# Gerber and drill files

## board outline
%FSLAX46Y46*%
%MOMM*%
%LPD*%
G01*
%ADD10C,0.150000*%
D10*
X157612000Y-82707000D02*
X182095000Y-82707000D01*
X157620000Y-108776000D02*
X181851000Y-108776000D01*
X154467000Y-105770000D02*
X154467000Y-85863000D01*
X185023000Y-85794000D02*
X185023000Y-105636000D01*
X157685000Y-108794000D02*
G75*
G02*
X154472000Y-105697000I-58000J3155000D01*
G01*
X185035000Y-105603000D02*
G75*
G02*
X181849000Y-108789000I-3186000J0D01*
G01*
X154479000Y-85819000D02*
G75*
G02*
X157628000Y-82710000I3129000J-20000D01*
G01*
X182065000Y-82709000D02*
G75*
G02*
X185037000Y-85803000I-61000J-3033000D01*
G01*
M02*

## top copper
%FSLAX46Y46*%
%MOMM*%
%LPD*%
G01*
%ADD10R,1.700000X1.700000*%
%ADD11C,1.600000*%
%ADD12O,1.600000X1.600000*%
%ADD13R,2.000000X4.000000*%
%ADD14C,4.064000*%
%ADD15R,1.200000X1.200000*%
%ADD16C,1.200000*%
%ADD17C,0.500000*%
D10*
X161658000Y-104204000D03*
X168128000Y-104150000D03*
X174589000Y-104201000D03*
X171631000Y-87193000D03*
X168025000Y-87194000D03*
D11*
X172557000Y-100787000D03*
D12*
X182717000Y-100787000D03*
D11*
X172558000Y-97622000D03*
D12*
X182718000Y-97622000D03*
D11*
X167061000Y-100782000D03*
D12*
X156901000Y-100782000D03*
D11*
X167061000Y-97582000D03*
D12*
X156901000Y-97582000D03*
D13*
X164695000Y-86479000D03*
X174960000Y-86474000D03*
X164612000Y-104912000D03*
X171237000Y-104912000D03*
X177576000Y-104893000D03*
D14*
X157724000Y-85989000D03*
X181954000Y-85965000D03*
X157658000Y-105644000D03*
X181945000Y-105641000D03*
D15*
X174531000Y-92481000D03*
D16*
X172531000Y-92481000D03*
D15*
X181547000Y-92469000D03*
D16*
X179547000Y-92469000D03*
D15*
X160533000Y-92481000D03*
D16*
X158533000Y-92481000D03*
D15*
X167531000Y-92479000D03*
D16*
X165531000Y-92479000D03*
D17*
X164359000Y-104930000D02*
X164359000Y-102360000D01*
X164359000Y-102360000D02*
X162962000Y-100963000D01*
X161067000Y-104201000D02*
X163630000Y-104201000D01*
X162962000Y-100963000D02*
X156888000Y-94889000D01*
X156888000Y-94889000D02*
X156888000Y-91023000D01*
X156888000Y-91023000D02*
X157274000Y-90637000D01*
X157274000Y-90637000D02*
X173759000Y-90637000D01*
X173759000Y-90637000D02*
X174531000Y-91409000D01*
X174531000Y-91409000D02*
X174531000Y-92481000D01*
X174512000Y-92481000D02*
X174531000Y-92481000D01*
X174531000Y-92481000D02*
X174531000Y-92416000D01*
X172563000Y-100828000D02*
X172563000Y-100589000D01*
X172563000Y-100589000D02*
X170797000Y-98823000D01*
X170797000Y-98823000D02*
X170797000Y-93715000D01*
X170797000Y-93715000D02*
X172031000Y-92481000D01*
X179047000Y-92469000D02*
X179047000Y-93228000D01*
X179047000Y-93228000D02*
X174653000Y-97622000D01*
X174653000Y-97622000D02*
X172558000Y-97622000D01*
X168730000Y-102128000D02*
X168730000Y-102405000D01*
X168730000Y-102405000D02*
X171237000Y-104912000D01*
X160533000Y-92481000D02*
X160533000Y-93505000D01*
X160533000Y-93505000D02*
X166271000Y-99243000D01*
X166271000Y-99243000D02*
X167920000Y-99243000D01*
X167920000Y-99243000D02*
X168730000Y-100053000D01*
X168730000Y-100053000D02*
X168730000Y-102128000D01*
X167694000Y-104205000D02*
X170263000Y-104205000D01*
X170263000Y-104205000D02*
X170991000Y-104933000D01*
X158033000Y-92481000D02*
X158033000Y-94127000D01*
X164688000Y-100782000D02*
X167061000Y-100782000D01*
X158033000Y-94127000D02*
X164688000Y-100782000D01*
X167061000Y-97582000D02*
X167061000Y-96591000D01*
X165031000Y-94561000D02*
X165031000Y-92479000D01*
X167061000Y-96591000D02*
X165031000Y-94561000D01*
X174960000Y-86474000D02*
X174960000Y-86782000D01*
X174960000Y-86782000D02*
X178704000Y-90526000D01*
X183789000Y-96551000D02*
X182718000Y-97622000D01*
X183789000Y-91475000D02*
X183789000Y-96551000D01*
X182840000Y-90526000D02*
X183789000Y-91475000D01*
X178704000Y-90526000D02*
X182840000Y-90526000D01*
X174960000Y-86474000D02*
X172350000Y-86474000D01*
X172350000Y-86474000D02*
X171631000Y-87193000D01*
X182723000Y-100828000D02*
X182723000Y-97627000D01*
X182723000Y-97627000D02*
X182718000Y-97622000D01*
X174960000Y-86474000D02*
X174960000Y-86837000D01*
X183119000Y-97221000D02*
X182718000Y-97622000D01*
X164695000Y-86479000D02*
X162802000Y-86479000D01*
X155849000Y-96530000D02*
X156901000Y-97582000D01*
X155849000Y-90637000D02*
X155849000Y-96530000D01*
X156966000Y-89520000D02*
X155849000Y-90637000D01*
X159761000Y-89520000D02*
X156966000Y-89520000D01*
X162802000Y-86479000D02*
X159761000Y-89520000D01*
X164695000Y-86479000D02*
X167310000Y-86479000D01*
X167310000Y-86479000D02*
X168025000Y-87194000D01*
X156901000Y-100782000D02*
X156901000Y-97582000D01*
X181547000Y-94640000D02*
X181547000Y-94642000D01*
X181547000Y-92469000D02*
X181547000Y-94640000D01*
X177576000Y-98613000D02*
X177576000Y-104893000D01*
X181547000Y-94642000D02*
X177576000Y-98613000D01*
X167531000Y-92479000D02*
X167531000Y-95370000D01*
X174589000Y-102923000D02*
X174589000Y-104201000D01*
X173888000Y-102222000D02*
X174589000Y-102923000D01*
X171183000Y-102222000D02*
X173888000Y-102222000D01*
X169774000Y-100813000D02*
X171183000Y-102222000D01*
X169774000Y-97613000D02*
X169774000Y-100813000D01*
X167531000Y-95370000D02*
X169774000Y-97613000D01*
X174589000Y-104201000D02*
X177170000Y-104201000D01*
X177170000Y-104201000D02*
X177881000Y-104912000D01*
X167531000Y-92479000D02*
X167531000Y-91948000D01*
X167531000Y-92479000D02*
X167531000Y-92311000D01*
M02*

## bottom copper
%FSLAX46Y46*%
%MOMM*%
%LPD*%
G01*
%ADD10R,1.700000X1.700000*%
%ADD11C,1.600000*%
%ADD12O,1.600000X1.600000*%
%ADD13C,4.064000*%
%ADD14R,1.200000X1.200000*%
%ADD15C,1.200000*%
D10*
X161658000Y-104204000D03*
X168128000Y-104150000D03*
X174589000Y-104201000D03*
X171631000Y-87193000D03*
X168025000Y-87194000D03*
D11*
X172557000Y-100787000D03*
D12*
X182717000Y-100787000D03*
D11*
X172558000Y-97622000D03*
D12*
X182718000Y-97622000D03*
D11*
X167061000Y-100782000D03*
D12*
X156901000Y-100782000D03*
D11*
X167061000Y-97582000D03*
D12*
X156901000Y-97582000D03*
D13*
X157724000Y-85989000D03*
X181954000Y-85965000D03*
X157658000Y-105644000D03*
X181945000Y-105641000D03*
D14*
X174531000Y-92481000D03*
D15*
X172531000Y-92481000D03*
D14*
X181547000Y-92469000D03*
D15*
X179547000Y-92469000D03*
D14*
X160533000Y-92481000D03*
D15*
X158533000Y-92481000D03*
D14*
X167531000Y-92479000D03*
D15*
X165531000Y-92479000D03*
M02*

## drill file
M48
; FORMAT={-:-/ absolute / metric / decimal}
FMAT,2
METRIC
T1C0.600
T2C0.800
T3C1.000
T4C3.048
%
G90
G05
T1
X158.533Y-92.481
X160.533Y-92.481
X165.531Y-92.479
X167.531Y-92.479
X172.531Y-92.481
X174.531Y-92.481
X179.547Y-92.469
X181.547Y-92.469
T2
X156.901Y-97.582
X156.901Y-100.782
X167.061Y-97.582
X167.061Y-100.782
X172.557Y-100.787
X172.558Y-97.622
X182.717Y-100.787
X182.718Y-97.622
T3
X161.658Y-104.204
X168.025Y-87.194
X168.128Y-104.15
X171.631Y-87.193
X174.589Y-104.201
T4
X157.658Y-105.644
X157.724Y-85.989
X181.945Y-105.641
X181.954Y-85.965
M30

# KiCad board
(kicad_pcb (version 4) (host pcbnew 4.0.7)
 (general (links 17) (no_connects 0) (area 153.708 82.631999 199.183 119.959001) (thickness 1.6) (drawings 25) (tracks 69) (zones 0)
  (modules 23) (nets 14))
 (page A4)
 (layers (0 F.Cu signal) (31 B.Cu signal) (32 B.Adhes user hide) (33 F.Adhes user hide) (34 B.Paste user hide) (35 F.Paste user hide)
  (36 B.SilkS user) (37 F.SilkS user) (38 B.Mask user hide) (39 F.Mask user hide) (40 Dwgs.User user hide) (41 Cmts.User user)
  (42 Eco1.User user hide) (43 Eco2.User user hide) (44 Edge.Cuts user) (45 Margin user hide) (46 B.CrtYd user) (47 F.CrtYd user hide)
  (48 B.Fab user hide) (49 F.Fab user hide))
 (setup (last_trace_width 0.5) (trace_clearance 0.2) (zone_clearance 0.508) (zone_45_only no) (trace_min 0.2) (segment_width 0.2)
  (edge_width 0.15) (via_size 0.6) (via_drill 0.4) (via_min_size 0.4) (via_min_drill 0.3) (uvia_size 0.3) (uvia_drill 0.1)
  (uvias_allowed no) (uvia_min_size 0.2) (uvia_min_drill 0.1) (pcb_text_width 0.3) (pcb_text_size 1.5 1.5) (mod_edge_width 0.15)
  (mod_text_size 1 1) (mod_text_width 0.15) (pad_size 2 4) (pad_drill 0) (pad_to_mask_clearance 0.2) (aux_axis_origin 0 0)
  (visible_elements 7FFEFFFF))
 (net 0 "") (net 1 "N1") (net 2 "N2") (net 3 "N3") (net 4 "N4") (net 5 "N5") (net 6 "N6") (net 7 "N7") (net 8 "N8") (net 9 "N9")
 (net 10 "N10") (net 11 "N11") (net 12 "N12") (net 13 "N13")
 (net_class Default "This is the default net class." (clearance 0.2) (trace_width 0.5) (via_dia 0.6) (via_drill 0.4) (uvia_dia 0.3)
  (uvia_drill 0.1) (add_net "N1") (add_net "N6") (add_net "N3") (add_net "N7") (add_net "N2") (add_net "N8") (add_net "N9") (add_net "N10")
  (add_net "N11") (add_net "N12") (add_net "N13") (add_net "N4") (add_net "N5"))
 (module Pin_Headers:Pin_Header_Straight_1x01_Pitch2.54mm (layer F.Cu) (at 161.658 104.204)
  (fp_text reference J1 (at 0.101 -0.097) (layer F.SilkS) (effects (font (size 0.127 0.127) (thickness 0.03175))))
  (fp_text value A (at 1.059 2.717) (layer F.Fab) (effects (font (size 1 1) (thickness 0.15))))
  (pad 1 thru_hole rect (at 0 0) (size 1.7 1.7) (drill 1) (layers *.Cu *.Mask) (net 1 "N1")))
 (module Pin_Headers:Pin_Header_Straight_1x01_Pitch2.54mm (layer F.Cu) (at 168.128 104.15)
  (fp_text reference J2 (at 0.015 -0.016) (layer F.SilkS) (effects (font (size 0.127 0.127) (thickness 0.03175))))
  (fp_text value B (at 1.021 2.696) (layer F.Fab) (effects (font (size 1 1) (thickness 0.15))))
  (pad 1 thru_hole rect (at 0 0) (size 1.7 1.7) (drill 1) (layers *.Cu *.Mask) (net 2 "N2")))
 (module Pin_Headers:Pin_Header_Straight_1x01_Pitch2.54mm (layer F.Cu) (at 174.589 104.201)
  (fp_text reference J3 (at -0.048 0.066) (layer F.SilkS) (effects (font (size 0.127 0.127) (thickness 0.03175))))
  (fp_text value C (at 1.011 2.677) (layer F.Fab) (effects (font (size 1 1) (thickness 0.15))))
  (pad 1 thru_hole rect (at 0 0) (size 1.7 1.7) (drill 1) (layers *.Cu *.Mask) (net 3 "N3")))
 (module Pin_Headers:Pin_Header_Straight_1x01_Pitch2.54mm (layer F.Cu) (at 171.631 87.193)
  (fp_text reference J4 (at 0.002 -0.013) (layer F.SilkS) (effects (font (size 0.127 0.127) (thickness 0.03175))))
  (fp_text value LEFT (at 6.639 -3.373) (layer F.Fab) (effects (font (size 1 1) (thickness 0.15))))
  (pad 1 thru_hole rect (at 0 0) (size 1.7 1.7) (drill 1) (layers *.Cu *.Mask) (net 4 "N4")))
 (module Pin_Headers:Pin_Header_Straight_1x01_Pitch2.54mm (layer F.Cu) (at 168.025 87.194)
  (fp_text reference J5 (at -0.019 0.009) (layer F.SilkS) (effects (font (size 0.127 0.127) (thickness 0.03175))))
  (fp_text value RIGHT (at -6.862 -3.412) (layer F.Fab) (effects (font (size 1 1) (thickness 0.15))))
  (pad 1 thru_hole rect (at 0 0) (size 1.7 1.7) (drill 1) (layers *.Cu *.Mask) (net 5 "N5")))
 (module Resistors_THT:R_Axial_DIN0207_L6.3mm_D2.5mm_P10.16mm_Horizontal (layer F.Cu) (at 172.557 100.787)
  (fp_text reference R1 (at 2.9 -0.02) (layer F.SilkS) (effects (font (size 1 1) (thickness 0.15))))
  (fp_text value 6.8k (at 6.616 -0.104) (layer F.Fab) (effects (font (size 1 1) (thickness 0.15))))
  (pad 1 thru_hole circle (at 0 0) (size 1.6 1.6) (drill 0.8) (layers *.Cu *.Mask) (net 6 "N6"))
  (pad 2 thru_hole oval (at 10.16 0) (size 1.6 1.6) (drill 0.8) (layers *.Cu *.Mask) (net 4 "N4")))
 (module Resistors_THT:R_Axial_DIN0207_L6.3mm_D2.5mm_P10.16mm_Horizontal (layer F.Cu) (at 172.558 97.622)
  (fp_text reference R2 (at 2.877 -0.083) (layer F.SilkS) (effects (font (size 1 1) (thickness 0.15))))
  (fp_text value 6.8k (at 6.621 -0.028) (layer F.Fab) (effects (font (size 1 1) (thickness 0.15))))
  (pad 1 thru_hole circle (at 0 0) (size 1.6 1.6) (drill 0.8) (layers *.Cu *.Mask) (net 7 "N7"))
  (pad 2 thru_hole oval (at 10.16 0) (size 1.6 1.6) (drill 0.8) (layers *.Cu *.Mask) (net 4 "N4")))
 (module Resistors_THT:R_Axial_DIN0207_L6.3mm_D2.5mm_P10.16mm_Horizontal (layer F.Cu) (at 167.061 100.782 180)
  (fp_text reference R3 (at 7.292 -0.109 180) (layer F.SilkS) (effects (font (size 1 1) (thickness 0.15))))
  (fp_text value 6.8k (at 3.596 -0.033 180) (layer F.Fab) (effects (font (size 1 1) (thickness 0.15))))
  (pad 1 thru_hole circle (at 0 0 180) (size 1.6 1.6) (drill 0.8) (layers *.Cu *.Mask) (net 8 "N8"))
  (pad 2 thru_hole oval (at 10.16 0 180) (size 1.6 1.6) (drill 0.8) (layers *.Cu *.Mask) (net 5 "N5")))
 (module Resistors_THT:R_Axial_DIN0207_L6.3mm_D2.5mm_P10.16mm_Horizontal (layer F.Cu) (at 167.061 97.582 180)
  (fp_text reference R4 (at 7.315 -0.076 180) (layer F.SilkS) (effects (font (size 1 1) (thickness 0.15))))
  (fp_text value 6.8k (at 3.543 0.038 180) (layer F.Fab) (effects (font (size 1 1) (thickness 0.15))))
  (pad 1 thru_hole circle (at 0 0 180) (size 1.6 1.6) (drill 0.8) (layers *.Cu *.Mask) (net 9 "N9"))
  (pad 2 thru_hole oval (at 10.16 0 180) (size 1.6 1.6) (drill 0.8) (layers *.Cu *.Mask) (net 5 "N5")))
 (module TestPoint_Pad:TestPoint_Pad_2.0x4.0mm (layer F.Cu) (at 164.695 86.479)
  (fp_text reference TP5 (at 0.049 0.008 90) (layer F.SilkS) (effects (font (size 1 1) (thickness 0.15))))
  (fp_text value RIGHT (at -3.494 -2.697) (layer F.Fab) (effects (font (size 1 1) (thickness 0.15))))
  (pad 1 smd rect (at 0 0) (size 2 4) (layers F.Cu F.Mask) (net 5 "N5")))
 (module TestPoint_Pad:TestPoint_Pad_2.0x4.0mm (layer F.Cu) (at 174.96 86.474)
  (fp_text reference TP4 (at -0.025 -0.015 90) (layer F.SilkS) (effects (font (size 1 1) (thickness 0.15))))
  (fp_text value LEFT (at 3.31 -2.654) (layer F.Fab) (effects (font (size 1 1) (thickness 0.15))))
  (pad 1 smd rect (at 0 0) (size 2 4) (layers F.Cu F.Mask) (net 4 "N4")))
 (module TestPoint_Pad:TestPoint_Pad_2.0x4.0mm (layer F.Cu) (at 164.612 104.912)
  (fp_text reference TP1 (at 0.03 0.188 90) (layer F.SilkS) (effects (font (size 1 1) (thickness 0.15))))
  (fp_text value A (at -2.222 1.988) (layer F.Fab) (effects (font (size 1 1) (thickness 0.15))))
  (pad 1 smd rect (at 0 0) (size 2 4) (layers F.Cu F.Mask) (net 1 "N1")))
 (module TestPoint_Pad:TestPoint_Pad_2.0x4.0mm (layer F.Cu) (at 171.237 104.912)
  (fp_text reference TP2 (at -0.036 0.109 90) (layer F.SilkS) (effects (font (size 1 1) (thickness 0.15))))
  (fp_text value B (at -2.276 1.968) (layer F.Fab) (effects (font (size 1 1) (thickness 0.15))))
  (pad 1 smd rect (at 0 0) (size 2 4) (layers F.Cu F.Mask) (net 2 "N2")))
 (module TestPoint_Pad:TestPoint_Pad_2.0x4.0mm (layer F.Cu) (at 177.576 104.893)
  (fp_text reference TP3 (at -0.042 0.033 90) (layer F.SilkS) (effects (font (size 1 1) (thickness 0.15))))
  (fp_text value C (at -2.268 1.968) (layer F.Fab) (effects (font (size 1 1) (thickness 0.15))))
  (pad 1 smd rect (at 0 0) (size 2 4) (layers F.Cu F.Mask) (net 3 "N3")))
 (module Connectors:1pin (layer F.Cu) (at 157.724 85.989)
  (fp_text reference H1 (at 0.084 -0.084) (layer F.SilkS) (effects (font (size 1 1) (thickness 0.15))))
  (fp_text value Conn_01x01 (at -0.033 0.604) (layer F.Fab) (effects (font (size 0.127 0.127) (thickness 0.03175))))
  (pad 1 thru_hole circle (at 0 0) (size 4.064 4.064) (drill 3.048) (layers *.Cu *.Mask) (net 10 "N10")))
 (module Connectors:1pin (layer F.Cu) (at 181.954 85.965)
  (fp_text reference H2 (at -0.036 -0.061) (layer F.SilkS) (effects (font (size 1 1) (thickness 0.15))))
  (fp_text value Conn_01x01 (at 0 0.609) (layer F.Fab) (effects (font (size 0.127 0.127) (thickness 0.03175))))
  (pad 1 thru_hole circle (at 0 0) (size 4.064 4.064) (drill 3.048) (layers *.Cu *.Mask) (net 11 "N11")))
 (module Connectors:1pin (layer F.Cu) (at 157.658 105.644)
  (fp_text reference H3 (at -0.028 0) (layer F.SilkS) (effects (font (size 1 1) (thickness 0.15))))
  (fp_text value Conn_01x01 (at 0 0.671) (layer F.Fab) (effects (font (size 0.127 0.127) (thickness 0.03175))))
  (pad 1 thru_hole circle (at 0 0) (size 4.064 4.064) (drill 3.048) (layers *.Cu *.Mask) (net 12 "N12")))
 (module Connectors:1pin (layer F.Cu) (at 181.945 105.641)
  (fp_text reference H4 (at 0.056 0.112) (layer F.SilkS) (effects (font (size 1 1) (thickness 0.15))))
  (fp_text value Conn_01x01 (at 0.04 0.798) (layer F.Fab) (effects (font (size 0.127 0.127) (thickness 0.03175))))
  (pad 1 thru_hole circle (at 0 0) (size 4.064 4.064) (drill 3.048) (layers *.Cu *.Mask) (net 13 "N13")))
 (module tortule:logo (layer B.Cu) (at 172.273 95.722 180)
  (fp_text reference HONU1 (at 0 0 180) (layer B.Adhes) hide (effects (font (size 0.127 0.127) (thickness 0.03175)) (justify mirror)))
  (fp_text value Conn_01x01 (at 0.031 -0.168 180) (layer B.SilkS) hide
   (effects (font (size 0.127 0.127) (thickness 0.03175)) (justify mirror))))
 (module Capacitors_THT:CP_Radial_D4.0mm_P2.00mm (layer F.Cu) (at 174.531 92.481 180)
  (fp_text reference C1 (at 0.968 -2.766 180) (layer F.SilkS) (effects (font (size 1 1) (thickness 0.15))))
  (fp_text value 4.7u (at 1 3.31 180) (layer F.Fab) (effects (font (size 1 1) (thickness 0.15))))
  (pad 1 thru_hole rect (at 0 0 180) (size 1.2 1.2) (drill 0.6) (layers *.Cu *.Mask) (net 1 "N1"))
  (pad 2 thru_hole circle (at 2 0 180) (size 1.2 1.2) (drill 0.6) (layers *.Cu *.Mask) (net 6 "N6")))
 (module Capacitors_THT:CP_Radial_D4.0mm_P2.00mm (layer F.Cu) (at 181.547 92.469 180)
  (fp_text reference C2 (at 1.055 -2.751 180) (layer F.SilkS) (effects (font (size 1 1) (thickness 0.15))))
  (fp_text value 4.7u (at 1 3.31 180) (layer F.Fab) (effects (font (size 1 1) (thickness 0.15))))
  (pad 1 thru_hole rect (at 0 0 180) (size 1.2 1.2) (drill 0.6) (layers *.Cu *.Mask) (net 3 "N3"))
  (pad 2 thru_hole circle (at 2 0 180) (size 1.2 1.2) (drill 0.6) (layers *.Cu *.Mask) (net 7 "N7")))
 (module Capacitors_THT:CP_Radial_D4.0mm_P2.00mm (layer F.Cu) (at 160.533 92.481 180)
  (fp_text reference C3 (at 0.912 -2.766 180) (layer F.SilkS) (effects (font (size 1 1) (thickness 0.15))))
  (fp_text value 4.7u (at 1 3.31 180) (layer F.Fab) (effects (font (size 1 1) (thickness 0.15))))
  (pad 1 thru_hole rect (at 0 0 180) (size 1.2 1.2) (drill 0.6) (layers *.Cu *.Mask) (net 2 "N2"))
  (pad 2 thru_hole circle (at 2 0 180) (size 1.2 1.2) (drill 0.6) (layers *.Cu *.Mask) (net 8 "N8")))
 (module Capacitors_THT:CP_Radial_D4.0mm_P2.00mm (layer F.Cu) (at 167.531 92.479 180)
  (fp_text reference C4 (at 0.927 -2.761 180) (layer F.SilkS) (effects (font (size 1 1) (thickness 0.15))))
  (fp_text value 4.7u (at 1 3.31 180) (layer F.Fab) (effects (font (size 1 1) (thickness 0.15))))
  (pad 1 thru_hole rect (at 0 0 180) (size 1.2 1.2) (drill 0.6) (layers *.Cu *.Mask) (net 3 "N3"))
  (pad 2 thru_hole circle (at 2 0 180) (size 1.2 1.2) (drill 0.6) (layers *.Cu *.Mask) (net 9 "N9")))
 (gr_line (start 157.612 82.707) (end 182.095 82.707) (angle 90) (layer Edge.Cuts) (width 0.15))
 (gr_line (start 157.62 108.776) (end 181.851 108.776) (angle 90) (layer Edge.Cuts) (width 0.15))
 (gr_line (start 154.467 105.77) (end 154.467 85.863) (angle 90) (layer Edge.Cuts) (width 0.15))
 (gr_line (start 185.023 85.794) (end 185.023 105.636) (angle 90) (layer Edge.Cuts) (width 0.15))
 (gr_arc (start 157.627 105.639) (end 157.685 108.794) (angle 90) (layer Edge.Cuts) (width 0.15))
 (gr_arc (start 181.849 105.603) (end 185.035 105.603) (angle 90) (layer Edge.Cuts) (width 0.15))
 (gr_arc (start 157.608 85.839) (end 154.479 85.819) (angle 90) (layer Edge.Cuts) (width 0.15))
 (gr_arc (start 182.004 85.742) (end 182.065 82.709) (angle 90) (layer Edge.Cuts) (width 0.15))
 (segment (start 164.359 104.93) (end 164.359 102.36) (width 0.5) (layer F.Cu) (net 1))
 (segment (start 164.359 102.36) (end 162.962 100.963) (width 0.5) (layer F.Cu) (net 1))
 (segment (start 161.067 104.201) (end 163.63 104.201) (width 0.5) (layer F.Cu) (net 1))
 (segment (start 162.962 100.963) (end 156.888 94.889) (width 0.5) (layer F.Cu) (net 1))
 (segment (start 156.888 94.889) (end 156.888 91.023) (width 0.5) (layer F.Cu) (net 1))
 (segment (start 156.888 91.023) (end 157.274 90.637) (width 0.5) (layer F.Cu) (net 1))
 (segment (start 157.274 90.637) (end 173.759 90.637) (width 0.5) (layer F.Cu) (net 1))
 (segment (start 173.759 90.637) (end 174.531 91.409) (width 0.5) (layer F.Cu) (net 1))
 (segment (start 174.531 91.409) (end 174.531 92.481) (width 0.5) (layer F.Cu) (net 1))
 (segment (start 174.512 92.481) (end 174.531 92.481) (width 0.5) (layer F.Cu) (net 1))
 (segment (start 174.531 92.481) (end 174.531 92.416) (width 0.5) (layer F.Cu) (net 1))
 (segment (start 172.563 100.828) (end 172.563 100.589) (width 0.5) (layer F.Cu) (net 6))
 (segment (start 172.563 100.589) (end 170.797 98.823) (width 0.5) (layer F.Cu) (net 6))
 (segment (start 170.797 98.823) (end 170.797 93.715) (width 0.5) (layer F.Cu) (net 6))
 (segment (start 170.797 93.715) (end 172.031 92.481) (width 0.5) (layer F.Cu) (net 6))
 (segment (start 179.047 92.469) (end 179.047 93.228) (width 0.5) (layer F.Cu) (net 7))
 (segment (start 179.047 93.228) (end 174.653 97.622) (width 0.5) (layer F.Cu) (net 7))
 (segment (start 174.653 97.622) (end 172.558 97.622) (width 0.5) (layer F.Cu) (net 7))
 (segment (start 168.73 102.128) (end 168.73 102.405) (width 0.5) (layer F.Cu) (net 2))
 (segment (start 168.73 102.405) (end 171.237 104.912) (width 0.5) (layer F.Cu) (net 2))
 (segment (start 160.533 92.481) (end 160.533 93.505) (width 0.5) (layer F.Cu) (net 2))
 (segment (start 160.533 93.505) (end 166.271 99.243) (width 0.5) (layer F.Cu) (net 2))
 (segment (start 166.271 99.243) (end 167.92 99.243) (width 0.5) (layer F.Cu) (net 2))
 (segment (start 167.92 99.243) (end 168.73 100.053) (width 0.5) (layer F.Cu) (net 2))
 (segment (start 168.73 100.053) (end 168.73 102.128) (width 0.5) (layer F.Cu) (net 2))
 (segment (start 167.694 104.205) (end 170.263 104.205) (width 0.5) (layer F.Cu) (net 2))
 (segment (start 170.263 104.205) (end 170.991 104.933) (width 0.5) (layer F.Cu) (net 2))
 (segment (start 158.033 92.481) (end 158.033 94.127) (width 0.5) (layer F.Cu) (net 8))
 (segment (start 164.688 100.782) (end 167.061 100.782) (width 0.5) (layer F.Cu) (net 8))
 (segment (start 158.033 94.127) (end 164.688 100.782) (width 0.5) (layer F.Cu) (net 8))
 (segment (start 167.061 97.582) (end 167.061 96.591) (width 0.5) (layer F.Cu) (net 9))
 (segment (start 165.031 94.561) (end 165.031 92.479) (width 0.5) (layer F.Cu) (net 9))
 (segment (start 167.061 96.591) (end 165.031 94.561) (width 0.5) (layer F.Cu) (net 9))
 (segment (start 174.96 86.474) (end 174.96 86.782) (width 0.5) (layer F.Cu) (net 4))
 (segment (start 174.96 86.782) (end 178.704 90.526) (width 0.5) (layer F.Cu) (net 4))
 (segment (start 183.789 96.551) (end 182.718 97.622) (width 0.5) (layer F.Cu) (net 4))
 (segment (start 183.789 91.475) (end 183.789 96.551) (width 0.5) (layer F.Cu) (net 4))
 (segment (start 182.84 90.526) (end 183.789 91.475) (width 0.5) (layer F.Cu) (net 4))
 (segment (start 178.704 90.526) (end 182.84 90.526) (width 0.5) (layer F.Cu) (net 4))
 (segment (start 174.96 86.474) (end 172.35 86.474) (width 0.5) (layer F.Cu) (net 4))
 (segment (start 172.35 86.474) (end 171.631 87.193) (width 0.5) (layer F.Cu) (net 4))
 (segment (start 182.723 100.828) (end 182.723 97.627) (width 0.5) (layer F.Cu) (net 4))
 (segment (start 182.723 97.627) (end 182.718 97.622) (width 0.5) (layer F.Cu) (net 4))
 (segment (start 174.96 86.474) (end 174.96 86.837) (width 0.5) (layer F.Cu) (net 4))
 (segment (start 183.119 97.221) (end 182.718 97.622) (width 0.5) (layer F.Cu) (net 4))
 (segment (start 164.695 86.479) (end 162.802 86.479) (width 0.5) (layer F.Cu) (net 5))
 (segment (start 155.849 96.53) (end 156.901 97.582) (width 0.5) (layer F.Cu) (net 5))
 (segment (start 155.849 90.637) (end 155.849 96.53) (width 0.5) (layer F.Cu) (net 5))
 (segment (start 156.966 89.52) (end 155.849 90.637) (width 0.5) (layer F.Cu) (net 5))
 (segment (start 159.761 89.52) (end 156.966 89.52) (width 0.5) (layer F.Cu) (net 5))
 (segment (start 162.802 86.479) (end 159.761 89.52) (width 0.5) (layer F.Cu) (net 5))
 (segment (start 164.695 86.479) (end 167.31 86.479) (width 0.5) (layer F.Cu) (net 5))
 (segment (start 167.31 86.479) (end 168.025 87.194) (width 0.5) (layer F.Cu) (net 5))
 (segment (start 156.901 100.782) (end 156.901 97.582) (width 0.5) (layer F.Cu) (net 5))
 (segment (start 181.547 94.64) (end 181.547 94.642) (width 0.5) (layer F.Cu) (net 3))
 (segment (start 181.547 92.469) (end 181.547 94.64) (width 0.5) (layer F.Cu) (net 3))
 (segment (start 177.576 98.613) (end 177.576 104.893) (width 0.5) (layer F.Cu) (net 3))
 (segment (start 181.547 94.642) (end 177.576 98.613) (width 0.5) (layer F.Cu) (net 3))
 (segment (start 167.531 92.479) (end 167.531 95.37) (width 0.5) (layer F.Cu) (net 3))
 (segment (start 174.589 102.923) (end 174.589 104.201) (width 0.5) (layer F.Cu) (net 3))
 (segment (start 173.888 102.222) (end 174.589 102.923) (width 0.5) (layer F.Cu) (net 3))
 (segment (start 171.183 102.222) (end 173.888 102.222) (width 0.5) (layer F.Cu) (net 3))
 (segment (start 169.774 100.813) (end 171.183 102.222) (width 0.5) (layer F.Cu) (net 3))
 (segment (start 169.774 97.613) (end 169.774 100.813) (width 0.5) (layer F.Cu) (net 3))
 (segment (start 167.531 95.37) (end 169.774 97.613) (width 0.5) (layer F.Cu) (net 3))
 (segment (start 174.589 104.201) (end 177.17 104.201) (width 0.5) (layer F.Cu) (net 3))
 (segment (start 177.17 104.201) (end 177.881 104.912) (width 0.5) (layer F.Cu) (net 3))
 (segment (start 167.531 92.479) (end 167.531 91.948) (width 0.5) (layer F.Cu) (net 3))
 (segment (start 167.531 92.479) (end 167.531 92.311) (width 0.5) (layer F.Cu) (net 3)))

